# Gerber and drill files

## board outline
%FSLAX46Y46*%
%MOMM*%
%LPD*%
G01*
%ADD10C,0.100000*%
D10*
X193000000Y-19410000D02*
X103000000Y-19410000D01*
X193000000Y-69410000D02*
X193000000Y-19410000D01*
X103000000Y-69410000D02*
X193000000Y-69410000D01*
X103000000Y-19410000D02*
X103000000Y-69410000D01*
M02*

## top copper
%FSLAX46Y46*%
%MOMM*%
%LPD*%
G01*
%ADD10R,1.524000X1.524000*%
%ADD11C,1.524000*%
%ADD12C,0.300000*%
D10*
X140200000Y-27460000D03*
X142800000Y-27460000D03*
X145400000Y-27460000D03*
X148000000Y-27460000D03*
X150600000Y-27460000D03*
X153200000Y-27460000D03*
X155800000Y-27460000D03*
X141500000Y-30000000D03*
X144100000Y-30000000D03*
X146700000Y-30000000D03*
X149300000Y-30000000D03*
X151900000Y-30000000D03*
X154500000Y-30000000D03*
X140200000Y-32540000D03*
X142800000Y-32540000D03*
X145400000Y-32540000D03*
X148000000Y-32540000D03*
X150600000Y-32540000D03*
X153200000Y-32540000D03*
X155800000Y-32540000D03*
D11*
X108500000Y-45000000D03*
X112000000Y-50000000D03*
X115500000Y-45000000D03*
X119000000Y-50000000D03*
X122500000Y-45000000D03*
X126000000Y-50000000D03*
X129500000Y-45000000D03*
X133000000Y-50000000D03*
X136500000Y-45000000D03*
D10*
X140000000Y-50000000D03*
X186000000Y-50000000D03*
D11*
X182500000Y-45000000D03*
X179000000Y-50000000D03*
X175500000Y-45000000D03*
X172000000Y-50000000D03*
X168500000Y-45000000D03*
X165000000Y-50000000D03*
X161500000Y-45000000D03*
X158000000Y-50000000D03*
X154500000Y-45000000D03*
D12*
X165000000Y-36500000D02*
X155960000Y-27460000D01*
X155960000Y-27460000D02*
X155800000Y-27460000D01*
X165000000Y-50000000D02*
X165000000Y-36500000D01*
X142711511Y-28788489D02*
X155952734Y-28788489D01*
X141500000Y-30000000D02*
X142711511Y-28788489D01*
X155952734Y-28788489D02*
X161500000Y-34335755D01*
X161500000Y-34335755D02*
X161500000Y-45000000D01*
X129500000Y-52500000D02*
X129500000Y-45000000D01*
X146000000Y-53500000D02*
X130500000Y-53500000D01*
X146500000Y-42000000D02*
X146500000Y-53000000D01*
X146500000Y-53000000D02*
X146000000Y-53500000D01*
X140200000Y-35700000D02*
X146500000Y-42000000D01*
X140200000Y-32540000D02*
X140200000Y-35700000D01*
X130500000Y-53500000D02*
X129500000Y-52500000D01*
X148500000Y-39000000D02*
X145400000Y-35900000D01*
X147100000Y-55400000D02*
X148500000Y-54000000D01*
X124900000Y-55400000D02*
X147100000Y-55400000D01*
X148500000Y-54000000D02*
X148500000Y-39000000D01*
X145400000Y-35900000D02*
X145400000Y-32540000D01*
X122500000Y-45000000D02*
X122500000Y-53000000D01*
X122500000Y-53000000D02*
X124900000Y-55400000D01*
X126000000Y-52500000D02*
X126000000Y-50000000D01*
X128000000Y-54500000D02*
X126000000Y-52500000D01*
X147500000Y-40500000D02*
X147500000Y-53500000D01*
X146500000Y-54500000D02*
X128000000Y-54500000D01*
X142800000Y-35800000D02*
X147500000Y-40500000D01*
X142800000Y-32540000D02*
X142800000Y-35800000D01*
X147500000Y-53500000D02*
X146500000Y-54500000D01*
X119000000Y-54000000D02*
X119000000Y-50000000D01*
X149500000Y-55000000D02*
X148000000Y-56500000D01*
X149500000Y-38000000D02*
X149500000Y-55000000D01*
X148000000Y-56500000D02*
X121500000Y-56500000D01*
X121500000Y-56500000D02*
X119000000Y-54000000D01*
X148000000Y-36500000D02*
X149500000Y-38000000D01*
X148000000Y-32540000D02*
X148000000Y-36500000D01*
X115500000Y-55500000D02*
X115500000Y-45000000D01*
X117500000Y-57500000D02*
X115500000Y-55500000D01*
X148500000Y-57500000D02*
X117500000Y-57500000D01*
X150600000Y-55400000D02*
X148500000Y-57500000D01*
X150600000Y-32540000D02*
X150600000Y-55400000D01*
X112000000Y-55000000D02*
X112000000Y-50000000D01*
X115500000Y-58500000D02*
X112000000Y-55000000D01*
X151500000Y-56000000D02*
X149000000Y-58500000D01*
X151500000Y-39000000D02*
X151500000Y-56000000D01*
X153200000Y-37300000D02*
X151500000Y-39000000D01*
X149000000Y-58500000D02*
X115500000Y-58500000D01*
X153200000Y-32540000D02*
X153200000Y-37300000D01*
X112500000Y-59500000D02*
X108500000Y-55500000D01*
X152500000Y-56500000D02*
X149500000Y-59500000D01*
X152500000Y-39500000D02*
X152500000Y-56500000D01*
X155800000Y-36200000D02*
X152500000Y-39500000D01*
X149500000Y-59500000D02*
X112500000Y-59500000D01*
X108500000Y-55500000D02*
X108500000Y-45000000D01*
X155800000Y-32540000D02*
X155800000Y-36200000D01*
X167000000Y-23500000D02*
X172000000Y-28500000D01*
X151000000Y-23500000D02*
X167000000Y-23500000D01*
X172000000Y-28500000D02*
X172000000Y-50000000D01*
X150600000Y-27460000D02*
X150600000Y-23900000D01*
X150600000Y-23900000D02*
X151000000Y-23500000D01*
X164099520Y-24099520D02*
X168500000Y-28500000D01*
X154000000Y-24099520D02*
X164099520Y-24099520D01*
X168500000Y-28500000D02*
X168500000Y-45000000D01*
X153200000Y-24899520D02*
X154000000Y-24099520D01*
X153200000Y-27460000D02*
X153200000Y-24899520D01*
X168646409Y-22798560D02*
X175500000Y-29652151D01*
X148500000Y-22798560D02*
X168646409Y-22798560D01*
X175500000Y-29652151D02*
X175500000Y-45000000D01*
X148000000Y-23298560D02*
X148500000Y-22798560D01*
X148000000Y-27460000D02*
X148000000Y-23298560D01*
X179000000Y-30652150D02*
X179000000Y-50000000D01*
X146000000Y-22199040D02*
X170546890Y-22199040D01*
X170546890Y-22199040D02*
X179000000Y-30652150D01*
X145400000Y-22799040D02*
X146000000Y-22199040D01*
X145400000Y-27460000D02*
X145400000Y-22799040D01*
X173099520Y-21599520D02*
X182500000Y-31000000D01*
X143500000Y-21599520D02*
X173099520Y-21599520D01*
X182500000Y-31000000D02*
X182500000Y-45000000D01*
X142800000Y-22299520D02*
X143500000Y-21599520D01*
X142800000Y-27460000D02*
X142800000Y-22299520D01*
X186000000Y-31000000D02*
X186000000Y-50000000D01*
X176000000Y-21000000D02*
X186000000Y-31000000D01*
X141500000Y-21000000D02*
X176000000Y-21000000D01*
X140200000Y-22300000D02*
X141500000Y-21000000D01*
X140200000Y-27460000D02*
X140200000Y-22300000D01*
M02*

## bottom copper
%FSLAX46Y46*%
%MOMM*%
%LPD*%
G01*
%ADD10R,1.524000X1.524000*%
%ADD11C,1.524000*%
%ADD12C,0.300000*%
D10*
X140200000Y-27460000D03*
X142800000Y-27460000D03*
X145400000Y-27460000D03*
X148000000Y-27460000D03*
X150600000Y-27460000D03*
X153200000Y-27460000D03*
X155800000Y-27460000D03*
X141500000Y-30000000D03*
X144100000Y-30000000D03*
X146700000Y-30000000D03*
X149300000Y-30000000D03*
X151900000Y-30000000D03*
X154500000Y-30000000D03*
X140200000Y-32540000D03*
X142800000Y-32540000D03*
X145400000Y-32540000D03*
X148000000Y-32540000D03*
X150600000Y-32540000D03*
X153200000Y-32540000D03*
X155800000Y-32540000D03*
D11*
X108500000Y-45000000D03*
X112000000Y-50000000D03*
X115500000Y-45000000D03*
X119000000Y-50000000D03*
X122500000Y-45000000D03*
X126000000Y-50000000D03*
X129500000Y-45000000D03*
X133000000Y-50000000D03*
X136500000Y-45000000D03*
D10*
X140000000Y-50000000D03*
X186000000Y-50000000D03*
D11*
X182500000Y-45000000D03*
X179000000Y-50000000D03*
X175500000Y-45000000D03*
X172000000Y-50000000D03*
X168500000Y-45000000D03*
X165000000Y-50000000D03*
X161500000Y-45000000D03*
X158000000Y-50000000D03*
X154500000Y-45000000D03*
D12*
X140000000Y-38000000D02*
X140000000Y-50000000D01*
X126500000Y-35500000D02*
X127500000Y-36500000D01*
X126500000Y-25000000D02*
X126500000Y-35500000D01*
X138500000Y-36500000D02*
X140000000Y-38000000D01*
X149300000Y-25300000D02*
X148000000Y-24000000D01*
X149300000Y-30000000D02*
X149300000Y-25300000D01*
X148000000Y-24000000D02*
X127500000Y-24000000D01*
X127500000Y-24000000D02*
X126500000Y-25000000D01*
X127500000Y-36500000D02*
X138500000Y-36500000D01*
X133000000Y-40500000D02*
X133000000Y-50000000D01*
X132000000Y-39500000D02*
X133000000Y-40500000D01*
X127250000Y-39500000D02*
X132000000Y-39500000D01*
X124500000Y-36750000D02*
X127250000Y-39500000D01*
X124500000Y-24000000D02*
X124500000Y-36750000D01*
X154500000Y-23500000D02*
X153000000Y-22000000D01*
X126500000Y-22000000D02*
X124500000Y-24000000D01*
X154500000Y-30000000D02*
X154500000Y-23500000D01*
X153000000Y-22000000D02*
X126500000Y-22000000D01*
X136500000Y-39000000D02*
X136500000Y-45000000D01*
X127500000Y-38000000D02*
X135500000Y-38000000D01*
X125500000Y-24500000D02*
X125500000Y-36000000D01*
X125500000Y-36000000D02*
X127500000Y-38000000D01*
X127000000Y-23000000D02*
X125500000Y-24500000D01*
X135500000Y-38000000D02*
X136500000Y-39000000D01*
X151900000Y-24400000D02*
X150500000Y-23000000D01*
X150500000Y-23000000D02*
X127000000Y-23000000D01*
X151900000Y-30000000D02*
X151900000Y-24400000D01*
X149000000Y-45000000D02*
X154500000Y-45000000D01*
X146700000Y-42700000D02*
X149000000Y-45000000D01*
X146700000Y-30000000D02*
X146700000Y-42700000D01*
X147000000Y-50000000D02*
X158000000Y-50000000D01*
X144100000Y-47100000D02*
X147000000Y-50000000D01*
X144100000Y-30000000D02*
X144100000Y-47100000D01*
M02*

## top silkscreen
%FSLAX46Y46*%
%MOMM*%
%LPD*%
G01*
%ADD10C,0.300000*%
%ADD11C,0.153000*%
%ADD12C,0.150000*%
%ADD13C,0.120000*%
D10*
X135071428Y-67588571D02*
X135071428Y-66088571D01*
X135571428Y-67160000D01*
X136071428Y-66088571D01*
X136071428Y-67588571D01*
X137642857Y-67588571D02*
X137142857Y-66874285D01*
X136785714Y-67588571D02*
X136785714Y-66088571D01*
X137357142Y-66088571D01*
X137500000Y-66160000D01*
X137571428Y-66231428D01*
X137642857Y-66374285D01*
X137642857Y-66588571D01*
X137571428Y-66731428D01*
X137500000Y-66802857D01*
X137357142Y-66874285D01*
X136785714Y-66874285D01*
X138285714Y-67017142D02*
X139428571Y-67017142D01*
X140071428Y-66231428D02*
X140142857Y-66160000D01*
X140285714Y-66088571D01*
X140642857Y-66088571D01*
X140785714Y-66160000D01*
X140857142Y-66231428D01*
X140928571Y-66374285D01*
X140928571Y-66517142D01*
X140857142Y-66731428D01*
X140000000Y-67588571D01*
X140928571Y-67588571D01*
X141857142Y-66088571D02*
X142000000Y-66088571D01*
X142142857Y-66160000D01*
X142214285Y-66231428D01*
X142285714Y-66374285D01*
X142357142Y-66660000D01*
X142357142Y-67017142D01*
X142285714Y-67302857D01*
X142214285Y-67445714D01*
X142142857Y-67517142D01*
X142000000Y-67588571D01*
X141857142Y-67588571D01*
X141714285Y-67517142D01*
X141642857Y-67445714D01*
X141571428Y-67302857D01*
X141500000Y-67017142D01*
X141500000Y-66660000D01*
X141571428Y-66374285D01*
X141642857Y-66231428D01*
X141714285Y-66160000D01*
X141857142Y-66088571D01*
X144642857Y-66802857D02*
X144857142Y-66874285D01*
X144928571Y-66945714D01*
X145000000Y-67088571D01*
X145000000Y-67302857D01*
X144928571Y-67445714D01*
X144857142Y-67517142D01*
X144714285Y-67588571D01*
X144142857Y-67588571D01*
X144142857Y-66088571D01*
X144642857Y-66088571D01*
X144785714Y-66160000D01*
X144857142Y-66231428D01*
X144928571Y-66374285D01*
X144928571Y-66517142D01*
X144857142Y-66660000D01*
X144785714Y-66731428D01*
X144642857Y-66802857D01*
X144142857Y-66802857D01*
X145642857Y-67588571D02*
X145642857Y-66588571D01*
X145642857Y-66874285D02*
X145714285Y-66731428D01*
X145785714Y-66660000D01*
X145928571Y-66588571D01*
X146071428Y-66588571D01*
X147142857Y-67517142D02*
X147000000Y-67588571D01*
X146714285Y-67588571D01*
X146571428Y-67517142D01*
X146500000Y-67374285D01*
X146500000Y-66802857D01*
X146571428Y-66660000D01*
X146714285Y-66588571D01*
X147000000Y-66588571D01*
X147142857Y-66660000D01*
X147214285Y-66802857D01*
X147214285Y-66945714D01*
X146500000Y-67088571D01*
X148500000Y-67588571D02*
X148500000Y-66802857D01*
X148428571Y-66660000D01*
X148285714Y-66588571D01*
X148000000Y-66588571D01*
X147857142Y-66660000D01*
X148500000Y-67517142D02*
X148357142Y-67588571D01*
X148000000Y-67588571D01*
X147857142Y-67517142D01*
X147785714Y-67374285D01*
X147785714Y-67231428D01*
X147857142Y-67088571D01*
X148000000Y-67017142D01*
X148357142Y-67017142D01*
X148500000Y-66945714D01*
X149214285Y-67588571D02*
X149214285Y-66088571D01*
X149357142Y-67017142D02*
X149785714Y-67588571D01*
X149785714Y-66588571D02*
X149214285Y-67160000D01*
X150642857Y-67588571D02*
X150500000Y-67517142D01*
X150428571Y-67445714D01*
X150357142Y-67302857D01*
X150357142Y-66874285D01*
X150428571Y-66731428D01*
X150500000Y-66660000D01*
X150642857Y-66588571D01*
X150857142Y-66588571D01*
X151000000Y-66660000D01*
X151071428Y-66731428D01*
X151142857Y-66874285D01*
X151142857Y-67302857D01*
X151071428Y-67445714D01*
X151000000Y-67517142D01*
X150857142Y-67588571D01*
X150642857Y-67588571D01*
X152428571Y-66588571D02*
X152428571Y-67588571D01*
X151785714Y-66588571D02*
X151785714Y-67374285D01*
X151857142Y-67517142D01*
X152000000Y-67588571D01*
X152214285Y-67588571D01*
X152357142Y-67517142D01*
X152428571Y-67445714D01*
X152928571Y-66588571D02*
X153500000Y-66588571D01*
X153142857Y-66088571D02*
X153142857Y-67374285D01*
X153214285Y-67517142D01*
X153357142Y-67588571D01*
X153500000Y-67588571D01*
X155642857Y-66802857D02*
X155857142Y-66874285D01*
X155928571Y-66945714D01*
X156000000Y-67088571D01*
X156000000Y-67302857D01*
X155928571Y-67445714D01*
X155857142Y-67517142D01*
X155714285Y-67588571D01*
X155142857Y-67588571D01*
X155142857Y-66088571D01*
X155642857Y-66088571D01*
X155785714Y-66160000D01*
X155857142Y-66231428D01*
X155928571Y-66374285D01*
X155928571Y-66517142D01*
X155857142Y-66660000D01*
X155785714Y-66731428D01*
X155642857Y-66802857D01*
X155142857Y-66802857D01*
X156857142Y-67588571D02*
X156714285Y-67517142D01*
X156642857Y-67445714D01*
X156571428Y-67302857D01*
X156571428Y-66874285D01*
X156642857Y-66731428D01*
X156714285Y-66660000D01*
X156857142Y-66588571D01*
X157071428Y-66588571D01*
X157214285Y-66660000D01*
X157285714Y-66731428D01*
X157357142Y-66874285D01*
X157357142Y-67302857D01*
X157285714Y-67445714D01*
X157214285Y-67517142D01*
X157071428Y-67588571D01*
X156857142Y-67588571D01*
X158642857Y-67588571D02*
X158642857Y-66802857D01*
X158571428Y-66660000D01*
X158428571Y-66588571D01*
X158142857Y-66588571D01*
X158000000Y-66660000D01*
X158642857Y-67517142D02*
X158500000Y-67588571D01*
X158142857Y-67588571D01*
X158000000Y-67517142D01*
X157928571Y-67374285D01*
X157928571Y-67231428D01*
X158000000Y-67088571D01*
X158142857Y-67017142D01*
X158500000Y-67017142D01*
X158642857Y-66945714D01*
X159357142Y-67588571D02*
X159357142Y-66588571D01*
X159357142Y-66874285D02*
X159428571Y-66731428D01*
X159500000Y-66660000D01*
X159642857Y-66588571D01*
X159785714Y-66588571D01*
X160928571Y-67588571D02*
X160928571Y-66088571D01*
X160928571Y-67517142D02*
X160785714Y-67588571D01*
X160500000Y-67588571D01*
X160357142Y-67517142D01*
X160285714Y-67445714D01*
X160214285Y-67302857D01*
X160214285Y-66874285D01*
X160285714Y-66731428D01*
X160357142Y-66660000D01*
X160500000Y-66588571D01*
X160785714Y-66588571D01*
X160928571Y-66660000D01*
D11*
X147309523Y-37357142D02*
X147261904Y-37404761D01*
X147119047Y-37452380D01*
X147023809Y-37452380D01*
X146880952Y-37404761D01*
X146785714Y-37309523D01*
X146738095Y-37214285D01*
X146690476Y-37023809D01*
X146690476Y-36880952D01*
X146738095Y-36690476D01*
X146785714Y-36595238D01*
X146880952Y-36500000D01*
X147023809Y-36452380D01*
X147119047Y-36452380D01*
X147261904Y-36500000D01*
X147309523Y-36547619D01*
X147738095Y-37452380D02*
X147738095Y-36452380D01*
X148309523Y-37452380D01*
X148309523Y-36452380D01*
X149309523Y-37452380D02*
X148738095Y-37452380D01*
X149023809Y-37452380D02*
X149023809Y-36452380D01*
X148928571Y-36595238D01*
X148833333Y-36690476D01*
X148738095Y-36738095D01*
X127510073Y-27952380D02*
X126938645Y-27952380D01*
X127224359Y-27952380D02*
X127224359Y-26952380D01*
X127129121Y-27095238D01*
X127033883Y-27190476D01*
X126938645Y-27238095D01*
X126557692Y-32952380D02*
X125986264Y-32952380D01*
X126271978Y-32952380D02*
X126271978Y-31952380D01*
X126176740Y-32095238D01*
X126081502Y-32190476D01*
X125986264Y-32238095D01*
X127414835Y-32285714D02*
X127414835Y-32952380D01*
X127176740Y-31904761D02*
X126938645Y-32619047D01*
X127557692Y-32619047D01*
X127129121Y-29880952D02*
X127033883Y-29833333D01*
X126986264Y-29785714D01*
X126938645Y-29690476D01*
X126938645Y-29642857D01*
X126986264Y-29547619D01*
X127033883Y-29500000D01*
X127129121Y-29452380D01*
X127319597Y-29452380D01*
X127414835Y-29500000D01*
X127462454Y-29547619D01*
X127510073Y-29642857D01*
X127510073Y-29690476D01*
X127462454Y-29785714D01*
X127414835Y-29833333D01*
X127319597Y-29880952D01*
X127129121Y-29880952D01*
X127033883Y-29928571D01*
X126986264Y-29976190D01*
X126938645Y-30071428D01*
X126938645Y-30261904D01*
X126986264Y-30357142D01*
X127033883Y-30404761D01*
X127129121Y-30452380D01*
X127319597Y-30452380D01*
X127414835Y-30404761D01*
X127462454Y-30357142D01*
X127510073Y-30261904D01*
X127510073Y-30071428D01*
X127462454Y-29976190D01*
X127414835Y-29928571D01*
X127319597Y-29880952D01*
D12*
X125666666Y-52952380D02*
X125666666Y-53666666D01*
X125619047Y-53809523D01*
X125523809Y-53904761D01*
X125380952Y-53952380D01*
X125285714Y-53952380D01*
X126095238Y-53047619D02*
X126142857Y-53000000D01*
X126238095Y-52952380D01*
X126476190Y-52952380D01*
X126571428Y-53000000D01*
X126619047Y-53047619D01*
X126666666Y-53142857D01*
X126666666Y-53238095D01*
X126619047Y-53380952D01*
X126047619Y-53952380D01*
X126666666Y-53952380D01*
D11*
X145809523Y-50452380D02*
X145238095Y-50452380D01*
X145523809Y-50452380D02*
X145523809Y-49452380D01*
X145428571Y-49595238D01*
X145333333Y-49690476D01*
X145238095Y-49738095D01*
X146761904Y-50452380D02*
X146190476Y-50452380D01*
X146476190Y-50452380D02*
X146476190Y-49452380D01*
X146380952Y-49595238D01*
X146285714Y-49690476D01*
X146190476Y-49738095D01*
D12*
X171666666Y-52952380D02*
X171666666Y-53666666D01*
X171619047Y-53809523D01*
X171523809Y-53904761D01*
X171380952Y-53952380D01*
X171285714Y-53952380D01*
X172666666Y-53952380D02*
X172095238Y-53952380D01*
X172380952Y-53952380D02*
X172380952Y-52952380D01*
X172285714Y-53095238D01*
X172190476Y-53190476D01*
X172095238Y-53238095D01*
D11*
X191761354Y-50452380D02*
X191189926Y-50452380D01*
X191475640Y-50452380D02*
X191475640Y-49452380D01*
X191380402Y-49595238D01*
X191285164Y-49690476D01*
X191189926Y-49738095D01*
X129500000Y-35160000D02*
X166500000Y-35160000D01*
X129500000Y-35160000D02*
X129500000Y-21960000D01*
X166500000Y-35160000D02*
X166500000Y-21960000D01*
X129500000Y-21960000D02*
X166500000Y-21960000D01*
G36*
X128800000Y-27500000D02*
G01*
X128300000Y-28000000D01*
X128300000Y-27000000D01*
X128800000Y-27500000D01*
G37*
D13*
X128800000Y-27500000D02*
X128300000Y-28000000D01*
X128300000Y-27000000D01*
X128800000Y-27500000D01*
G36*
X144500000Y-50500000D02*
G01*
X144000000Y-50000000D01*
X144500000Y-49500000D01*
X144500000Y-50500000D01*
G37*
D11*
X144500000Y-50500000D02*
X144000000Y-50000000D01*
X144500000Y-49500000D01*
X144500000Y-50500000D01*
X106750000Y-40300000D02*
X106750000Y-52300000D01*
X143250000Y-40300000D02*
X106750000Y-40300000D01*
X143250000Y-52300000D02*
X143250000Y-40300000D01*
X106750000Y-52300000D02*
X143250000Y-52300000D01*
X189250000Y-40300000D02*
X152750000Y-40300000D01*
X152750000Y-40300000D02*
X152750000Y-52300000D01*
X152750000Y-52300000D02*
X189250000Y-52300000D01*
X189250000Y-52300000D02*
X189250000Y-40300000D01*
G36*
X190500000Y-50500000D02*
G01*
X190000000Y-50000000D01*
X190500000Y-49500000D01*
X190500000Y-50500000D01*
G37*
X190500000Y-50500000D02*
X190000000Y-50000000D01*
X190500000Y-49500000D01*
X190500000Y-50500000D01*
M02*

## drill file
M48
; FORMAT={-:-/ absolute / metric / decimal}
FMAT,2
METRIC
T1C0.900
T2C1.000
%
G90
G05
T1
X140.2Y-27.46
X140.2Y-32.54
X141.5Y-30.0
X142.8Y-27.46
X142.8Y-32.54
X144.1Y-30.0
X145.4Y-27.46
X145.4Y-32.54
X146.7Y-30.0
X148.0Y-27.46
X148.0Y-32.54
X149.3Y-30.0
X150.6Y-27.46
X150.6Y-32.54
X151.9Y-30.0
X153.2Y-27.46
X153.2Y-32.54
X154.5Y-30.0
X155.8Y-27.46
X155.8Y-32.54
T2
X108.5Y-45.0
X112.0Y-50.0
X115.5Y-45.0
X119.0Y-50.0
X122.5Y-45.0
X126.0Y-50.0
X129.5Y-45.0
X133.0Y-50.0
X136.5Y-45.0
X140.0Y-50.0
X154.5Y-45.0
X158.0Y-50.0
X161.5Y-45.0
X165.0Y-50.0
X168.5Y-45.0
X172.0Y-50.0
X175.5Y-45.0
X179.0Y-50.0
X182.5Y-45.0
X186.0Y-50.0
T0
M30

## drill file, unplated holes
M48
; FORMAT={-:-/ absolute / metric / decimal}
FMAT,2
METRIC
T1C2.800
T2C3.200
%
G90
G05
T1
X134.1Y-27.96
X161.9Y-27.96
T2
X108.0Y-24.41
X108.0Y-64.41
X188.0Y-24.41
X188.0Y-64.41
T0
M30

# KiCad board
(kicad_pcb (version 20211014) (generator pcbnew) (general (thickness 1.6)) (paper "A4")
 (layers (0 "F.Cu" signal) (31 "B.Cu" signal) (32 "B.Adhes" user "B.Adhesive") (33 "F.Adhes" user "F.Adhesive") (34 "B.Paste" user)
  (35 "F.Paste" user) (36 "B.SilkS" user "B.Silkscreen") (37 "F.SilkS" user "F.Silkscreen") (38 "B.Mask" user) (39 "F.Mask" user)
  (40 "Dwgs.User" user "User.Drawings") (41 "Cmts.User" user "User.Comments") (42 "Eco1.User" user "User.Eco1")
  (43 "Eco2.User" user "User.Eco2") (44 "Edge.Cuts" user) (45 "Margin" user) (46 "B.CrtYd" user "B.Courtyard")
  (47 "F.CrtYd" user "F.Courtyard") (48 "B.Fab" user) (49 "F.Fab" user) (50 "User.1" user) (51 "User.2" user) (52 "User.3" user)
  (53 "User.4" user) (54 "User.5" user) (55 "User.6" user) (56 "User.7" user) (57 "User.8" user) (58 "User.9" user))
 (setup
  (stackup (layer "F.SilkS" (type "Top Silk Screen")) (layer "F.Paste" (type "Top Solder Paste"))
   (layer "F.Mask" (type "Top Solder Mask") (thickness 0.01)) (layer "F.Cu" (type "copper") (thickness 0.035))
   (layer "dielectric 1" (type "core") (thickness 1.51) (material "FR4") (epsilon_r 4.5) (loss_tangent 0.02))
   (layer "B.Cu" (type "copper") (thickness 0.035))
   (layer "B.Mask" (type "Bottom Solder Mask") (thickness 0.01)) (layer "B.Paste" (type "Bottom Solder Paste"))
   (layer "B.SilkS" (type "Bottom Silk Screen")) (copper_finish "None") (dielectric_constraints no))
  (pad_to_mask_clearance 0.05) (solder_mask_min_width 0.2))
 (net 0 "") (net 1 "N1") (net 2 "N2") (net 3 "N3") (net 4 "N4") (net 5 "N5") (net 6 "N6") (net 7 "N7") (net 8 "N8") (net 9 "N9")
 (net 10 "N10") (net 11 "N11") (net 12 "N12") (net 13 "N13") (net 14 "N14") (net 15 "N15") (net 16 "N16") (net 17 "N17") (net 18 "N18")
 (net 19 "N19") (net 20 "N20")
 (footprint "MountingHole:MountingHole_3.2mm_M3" (layer "F.Cu") (at 188 64.41)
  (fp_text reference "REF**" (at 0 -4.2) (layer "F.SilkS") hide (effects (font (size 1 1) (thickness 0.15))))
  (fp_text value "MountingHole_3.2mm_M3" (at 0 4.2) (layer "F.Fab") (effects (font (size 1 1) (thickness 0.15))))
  (pad "" np_thru_hole circle (at 0 0) (size 3.2 3.2) (drill 3.2) (layers *.Cu *.Mask)))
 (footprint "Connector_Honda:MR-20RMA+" (layer "F.Cu") (at 148 30)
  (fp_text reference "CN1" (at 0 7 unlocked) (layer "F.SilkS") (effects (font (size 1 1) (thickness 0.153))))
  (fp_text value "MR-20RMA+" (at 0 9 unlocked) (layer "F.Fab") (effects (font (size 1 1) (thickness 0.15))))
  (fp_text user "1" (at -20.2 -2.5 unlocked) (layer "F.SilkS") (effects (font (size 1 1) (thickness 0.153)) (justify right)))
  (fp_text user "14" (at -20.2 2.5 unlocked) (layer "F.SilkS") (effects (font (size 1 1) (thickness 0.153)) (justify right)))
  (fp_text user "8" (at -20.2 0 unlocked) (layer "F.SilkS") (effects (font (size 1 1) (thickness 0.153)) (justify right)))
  (fp_line (start -18.5 5.16) (end 18.5 5.16) (layer "F.SilkS") (width 0.153))
  (fp_line (start -18.5 5.16) (end -18.5 -8.04) (layer "F.SilkS") (width 0.153))
  (fp_line (start 18.5 5.16) (end 18.5 -8.04) (layer "F.SilkS") (width 0.153))
  (fp_line (start -18.5 -8.04) (end 18.5 -8.04) (layer "F.SilkS") (width 0.153))
  (fp_poly (pts (xy -19.2 -2.5) (xy -19.7 -2) (xy -19.7 -3)) (layer "F.SilkS") (width 0.12) (fill solid))
  (pad "" np_thru_hole circle (at -13.9 -2.04) (size 2.8 2.8) (drill 2.8) (layers F&B.Cu *.Mask))
  (pad "" np_thru_hole circle (at 13.9 -2.04) (size 2.8 2.8) (drill 2.8) (layers F&B.Cu *.Mask))
  (pad "1" thru_hole rect (at -7.8 -2.54) (size 1.524 1.524) (drill 0.9) (layers *.Cu *.Mask) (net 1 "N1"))
  (pad "2" thru_hole rect (at -5.2 -2.54) (size 1.524 1.524) (drill 0.9) (layers *.Cu *.Mask) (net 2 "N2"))
  (pad "3" thru_hole rect (at -2.6 -2.54) (size 1.524 1.524) (drill 0.9) (layers *.Cu *.Mask) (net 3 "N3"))
  (pad "4" thru_hole rect (at 0 -2.54) (size 1.524 1.524) (drill 0.9) (layers *.Cu *.Mask) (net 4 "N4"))
  (pad "5" thru_hole rect (at 2.6 -2.54) (size 1.524 1.524) (drill 0.9) (layers *.Cu *.Mask) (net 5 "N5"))
  (pad "6" thru_hole rect (at 5.2 -2.54) (size 1.524 1.524) (drill 0.9) (layers *.Cu *.Mask) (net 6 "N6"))
  (pad "7" thru_hole rect (at 7.8 -2.54) (size 1.524 1.524) (drill 0.9) (layers *.Cu *.Mask) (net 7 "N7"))
  (pad "8" thru_hole rect (at -6.5 0) (size 1.524 1.524) (drill 0.9) (layers *.Cu *.Mask) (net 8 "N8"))
  (pad "9" thru_hole rect (at -3.9 0) (size 1.524 1.524) (drill 0.9) (layers *.Cu *.Mask) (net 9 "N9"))
  (pad "10" thru_hole rect (at -1.3 0) (size 1.524 1.524) (drill 0.9) (layers *.Cu *.Mask) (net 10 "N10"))
  (pad "11" thru_hole rect (at 1.3 0) (size 1.524 1.524) (drill 0.9) (layers *.Cu *.Mask) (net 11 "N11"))
  (pad "12" thru_hole rect (at 3.9 0) (size 1.524 1.524) (drill 0.9) (layers *.Cu *.Mask) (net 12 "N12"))
  (pad "13" thru_hole rect (at 6.5 0) (size 1.524 1.524) (drill 0.9) (layers *.Cu *.Mask) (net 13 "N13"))
  (pad "14" thru_hole rect (at -7.8 2.54) (size 1.524 1.524) (drill 0.9) (layers *.Cu *.Mask) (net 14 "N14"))
  (pad "15" thru_hole rect (at -5.2 2.54) (size 1.524 1.524) (drill 0.9) (layers *.Cu *.Mask) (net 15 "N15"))
  (pad "16" thru_hole rect (at -2.6 2.54) (size 1.524 1.524) (drill 0.9) (layers *.Cu *.Mask) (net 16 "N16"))
  (pad "17" thru_hole rect (at 0 2.54) (size 1.524 1.524) (drill 0.9) (layers *.Cu *.Mask) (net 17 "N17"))
  (pad "18" thru_hole rect (at 2.6 2.54) (size 1.524 1.524) (drill 0.9) (layers *.Cu *.Mask) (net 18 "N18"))
  (pad "19" thru_hole rect (at 5.2 2.54) (size 1.524 1.524) (drill 0.9) (layers *.Cu *.Mask) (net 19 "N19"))
  (pad "20" thru_hole rect (at 7.8 2.54) (size 1.524 1.524) (drill 0.9) (layers *.Cu *.Mask) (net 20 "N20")))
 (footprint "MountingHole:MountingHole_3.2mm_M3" (layer "F.Cu") (at 108 64.41)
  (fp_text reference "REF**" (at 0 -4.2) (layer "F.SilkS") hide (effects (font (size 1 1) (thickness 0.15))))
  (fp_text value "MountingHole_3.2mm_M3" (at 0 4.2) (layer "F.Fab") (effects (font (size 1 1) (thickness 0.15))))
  (pad "" np_thru_hole circle (at 0 0) (size 3.2 3.2) (drill 3.2) (layers *.Cu *.Mask)))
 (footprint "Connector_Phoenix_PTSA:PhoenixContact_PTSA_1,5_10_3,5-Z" (layer "F.Cu") (at 140 50 180)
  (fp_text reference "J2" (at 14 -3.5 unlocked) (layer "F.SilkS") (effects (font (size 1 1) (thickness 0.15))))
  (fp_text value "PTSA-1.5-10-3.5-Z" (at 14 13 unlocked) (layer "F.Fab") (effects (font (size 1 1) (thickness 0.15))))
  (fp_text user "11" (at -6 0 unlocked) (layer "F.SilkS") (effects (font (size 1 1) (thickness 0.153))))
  (fp_line (start 33.25 -2.3) (end -3.25 -2.3) (layer "F.SilkS") (width 0.153))
  (fp_line (start -3.25 -2.3) (end -3.25 9.7) (layer "F.SilkS") (width 0.153))
  (fp_line (start -3.25 9.7) (end 33.25 9.7) (layer "F.SilkS") (width 0.153))
  (fp_line (start 33.25 9.7) (end 33.25 -2.3) (layer "F.SilkS") (width 0.153))
  (fp_poly (pts (xy -4 0) (xy -4.5 0.5) (xy -4.5 -0.5)) (layer "F.SilkS") (width 0.153) (fill solid))
  (pad "1" thru_hole rect (at 0 0 180) (size 1.524 1.524) (drill 1) (layers *.Cu *.Mask) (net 11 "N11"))
  (pad "2" thru_hole circle (at 3.5 5 180) (size 1.524 1.524) (drill 1) (layers *.Cu *.Mask) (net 12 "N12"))
  (pad "3" thru_hole circle (at 7 0 180) (size 1.524 1.524) (drill 1) (layers *.Cu *.Mask) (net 13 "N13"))
  (pad "4" thru_hole circle (at 10.5 5 180) (size 1.524 1.524) (drill 1) (layers *.Cu *.Mask) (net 14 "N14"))
  (pad "5" thru_hole circle (at 14 0 180) (size 1.524 1.524) (drill 1) (layers *.Cu *.Mask) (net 15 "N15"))
  (pad "6" thru_hole circle (at 17.5 5 180) (size 1.524 1.524) (drill 1) (layers *.Cu *.Mask) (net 16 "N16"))
  (pad "7" thru_hole circle (at 21 0 180) (size 1.524 1.524) (drill 1) (layers *.Cu *.Mask) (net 17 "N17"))
  (pad "8" thru_hole circle (at 24.5 5 180) (size 1.524 1.524) (drill 1) (layers *.Cu *.Mask) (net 18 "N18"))
  (pad "9" thru_hole circle (at 28 0 180) (size 1.524 1.524) (drill 1) (layers *.Cu *.Mask) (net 19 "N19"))
  (pad "10" thru_hole circle (at 31.5 5 180) (size 1.524 1.524) (drill 1) (layers *.Cu *.Mask) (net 20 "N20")))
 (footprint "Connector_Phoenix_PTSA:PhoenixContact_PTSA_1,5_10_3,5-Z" (layer "F.Cu") (at 186 50 180)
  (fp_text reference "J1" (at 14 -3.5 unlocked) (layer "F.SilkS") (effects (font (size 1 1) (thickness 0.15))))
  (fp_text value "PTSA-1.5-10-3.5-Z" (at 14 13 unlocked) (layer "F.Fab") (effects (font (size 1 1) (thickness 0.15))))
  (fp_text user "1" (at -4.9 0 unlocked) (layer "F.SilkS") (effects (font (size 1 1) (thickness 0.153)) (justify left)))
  (fp_line (start -3.25 9.7) (end 33.25 9.7) (layer "F.SilkS") (width 0.153))
  (fp_line (start 33.25 9.7) (end 33.25 -2.3) (layer "F.SilkS") (width 0.153))
  (fp_line (start 33.25 -2.3) (end -3.25 -2.3) (layer "F.SilkS") (width 0.153))
  (fp_line (start -3.25 -2.3) (end -3.25 9.7) (layer "F.SilkS") (width 0.153))
  (fp_poly (pts (xy -4 0) (xy -4.5 0.5) (xy -4.5 -0.5)) (layer "F.SilkS") (width 0.153) (fill solid))
  (pad "1" thru_hole rect (at 0 0 180) (size 1.524 1.524) (drill 1) (layers *.Cu *.Mask) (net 1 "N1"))
  (pad "2" thru_hole circle (at 3.5 5 180) (size 1.524 1.524) (drill 1) (layers *.Cu *.Mask) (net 2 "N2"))
  (pad "3" thru_hole circle (at 7 0 180) (size 1.524 1.524) (drill 1) (layers *.Cu *.Mask) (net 3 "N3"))
  (pad "4" thru_hole circle (at 10.5 5 180) (size 1.524 1.524) (drill 1) (layers *.Cu *.Mask) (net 4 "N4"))
  (pad "5" thru_hole circle (at 14 0 180) (size 1.524 1.524) (drill 1) (layers *.Cu *.Mask) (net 5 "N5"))
  (pad "6" thru_hole circle (at 17.5 5 180) (size 1.524 1.524) (drill 1) (layers *.Cu *.Mask) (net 6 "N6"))
  (pad "7" thru_hole circle (at 21 0 180) (size 1.524 1.524) (drill 1) (layers *.Cu *.Mask) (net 7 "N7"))
  (pad "8" thru_hole circle (at 24.5 5 180) (size 1.524 1.524) (drill 1) (layers *.Cu *.Mask) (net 8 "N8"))
  (pad "9" thru_hole circle (at 28 0 180) (size 1.524 1.524) (drill 1) (layers *.Cu *.Mask) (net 9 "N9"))
  (pad "10" thru_hole circle (at 31.5 5 180) (size 1.524 1.524) (drill 1) (layers *.Cu *.Mask) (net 10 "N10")))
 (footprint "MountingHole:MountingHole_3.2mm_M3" (layer "F.Cu") (at 188 24.41)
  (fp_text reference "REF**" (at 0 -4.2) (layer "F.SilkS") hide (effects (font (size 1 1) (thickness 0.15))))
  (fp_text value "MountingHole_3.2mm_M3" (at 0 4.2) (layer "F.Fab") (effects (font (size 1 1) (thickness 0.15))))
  (pad "" np_thru_hole circle (at 0 0) (size 3.2 3.2) (drill 3.2) (layers *.Cu *.Mask)))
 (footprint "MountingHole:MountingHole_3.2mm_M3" (layer "F.Cu") (at 108 24.41)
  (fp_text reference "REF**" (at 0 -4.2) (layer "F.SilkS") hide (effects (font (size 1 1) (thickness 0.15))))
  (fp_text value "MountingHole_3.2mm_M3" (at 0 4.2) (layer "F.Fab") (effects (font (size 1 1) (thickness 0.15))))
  (pad "" np_thru_hole circle (at 0 0) (size 3.2 3.2) (drill 3.2) (layers *.Cu *.Mask)))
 (gr_line (start 193 19.41) (end 103 19.41) (layer "Edge.Cuts") (width 0.1))
 (gr_line (start 193 69.41) (end 193 19.41) (layer "Edge.Cuts") (width 0.1))
 (gr_line (start 103 69.41) (end 193 69.41) (layer "Edge.Cuts") (width 0.1))
 (gr_line (start 103 19.41) (end 103 69.41) (layer "Edge.Cuts") (width 0.1))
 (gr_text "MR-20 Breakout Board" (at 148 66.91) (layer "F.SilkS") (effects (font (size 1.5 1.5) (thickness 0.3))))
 (segment (start 186 31) (end 186 50) (width 0.3) (layer "F.Cu") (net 1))
 (segment (start 176 21) (end 186 31) (width 0.3) (layer "F.Cu") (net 1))
 (segment (start 140.2 22.3) (end 141.5 21) (width 0.3) (layer "F.Cu") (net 1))
 (segment (start 140.2 27.46) (end 140.2 22.3) (width 0.3) (layer "F.Cu") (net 1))
 (segment (start 141.5 21) (end 176 21) (width 0.3) (layer "F.Cu") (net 1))
 (segment (start 173.09952 21.59952) (end 182.5 31) (width 0.3) (layer "F.Cu") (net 2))
 (segment (start 142.8 22.29952) (end 143.5 21.59952) (width 0.3) (layer "F.Cu") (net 2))
 (segment (start 143.5 21.59952) (end 173.09952 21.59952) (width 0.3) (layer "F.Cu") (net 2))
 (segment (start 182.5 31) (end 182.5 45) (width 0.3) (layer "F.Cu") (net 2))
 (segment (start 142.8 27.46) (end 142.8 22.29952) (width 0.3) (layer "F.Cu") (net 2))
 (segment (start 145.4 27.46) (end 145.4 22.79904) (width 0.3) (layer "F.Cu") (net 3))
 (segment (start 146 22.19904) (end 170.54689 22.19904) (width 0.3) (layer "F.Cu") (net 3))
 (segment (start 145.4 22.79904) (end 146 22.19904) (width 0.3) (layer "F.Cu") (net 3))
 (segment (start 170.54689 22.19904) (end 179 30.65215) (width 0.3) (layer "F.Cu") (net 3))
 (segment (start 179 30.65215) (end 179 50) (width 0.3) (layer "F.Cu") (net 3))
 (segment (start 148.5 22.79856) (end 168.646409 22.79856) (width 0.3) (layer "F.Cu") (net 4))
 (segment (start 148 23.29856) (end 148.5 22.79856) (width 0.3) (layer "F.Cu") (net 4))
 (segment (start 148 27.46) (end 148 23.29856) (width 0.3) (layer "F.Cu") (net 4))
 (segment (start 175.5 29.652151) (end 175.5 45) (width 0.3) (layer "F.Cu") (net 4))
 (segment (start 168.646409 22.79856) (end 175.5 29.652151) (width 0.3) (layer "F.Cu") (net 4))
 (segment (start 150.6 23.9) (end 151 23.5) (width 0.3) (layer "F.Cu") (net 5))
 (segment (start 172 28.5) (end 172 50) (width 0.3) (layer "F.Cu") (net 5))
 (segment (start 167 23.5) (end 172 28.5) (width 0.3) (layer "F.Cu") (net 5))
 (segment (start 150.6 27.46) (end 150.6 23.9) (width 0.3) (layer "F.Cu") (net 5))
 (segment (start 151 23.5) (end 167 23.5) (width 0.3) (layer "F.Cu") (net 5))
 (segment (start 153.2 27.46) (end 153.2 24.89952) (width 0.3) (layer "F.Cu") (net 6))
 (segment (start 168.5 28.5) (end 168.5 45) (width 0.3) (layer "F.Cu") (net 6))
 (segment (start 164.09952 24.09952) (end 168.5 28.5) (width 0.3) (layer "F.Cu") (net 6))
 (segment (start 154 24.09952) (end 164.09952 24.09952) (width 0.3) (layer "F.Cu") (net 6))
 (segment (start 153.2 24.89952) (end 154 24.09952) (width 0.3) (layer "F.Cu") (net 6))
 (segment (start 155.96 27.46) (end 155.8 27.46) (width 0.3) (layer "F.Cu") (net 7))
 (segment (start 165 50) (end 165 36.5) (width 0.3) (layer "F.Cu") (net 7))
 (segment (start 165 36.5) (end 155.96 27.46) (width 0.3) (layer "F.Cu") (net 7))
 (segment (start 161.5 34.335755) (end 161.5 45) (width 0.3) (layer "F.Cu") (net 8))
 (segment (start 141.5 30) (end 142.711511 28.788489) (width 0.3) (layer "F.Cu") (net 8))
 (segment (start 142.711511 28.788489) (end 155.952734 28.788489) (width 0.3) (layer "F.Cu") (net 8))
 (segment (start 155.952734 28.788489) (end 161.5 34.335755) (width 0.3) (layer "F.Cu") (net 8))
 (segment (start 144.1 47.1) (end 147 50) (width 0.3) (layer "B.Cu") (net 9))
 (segment (start 144.1 30) (end 144.1 47.1) (width 0.3) (layer "B.Cu") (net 9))
 (segment (start 147 50) (end 158 50) (width 0.3) (layer "B.Cu") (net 9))
 (segment (start 146.7 30) (end 146.7 42.7) (width 0.3) (layer "B.Cu") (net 10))
 (segment (start 149 45) (end 154.5 45) (width 0.3) (layer "B.Cu") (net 10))
 (segment (start 146.7 42.7) (end 149 45) (width 0.3) (layer "B.Cu") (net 10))
 (segment (start 127.5 24) (end 126.5 25) (width 0.3) (layer "B.Cu") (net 11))
 (segment (start 149.3 30) (end 149.3 25.3) (width 0.3) (layer "B.Cu") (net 11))
 (segment (start 126.5 25) (end 126.5 35.5) (width 0.3) (layer "B.Cu") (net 11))
 (segment (start 126.5 35.5) (end 127.5 36.5) (width 0.3) (layer "B.Cu") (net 11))
 (segment (start 140 38) (end 140 50) (width 0.3) (layer "B.Cu") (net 11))
 (segment (start 148 24) (end 127.5 24) (width 0.3) (layer "B.Cu") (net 11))
 (segment (start 138.5 36.5) (end 140 38) (width 0.3) (layer "B.Cu") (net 11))
 (segment (start 127.5 36.5) (end 138.5 36.5) (width 0.3) (layer "B.Cu") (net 11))
 (segment (start 149.3 25.3) (end 148 24) (width 0.3) (layer "B.Cu") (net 11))
 (segment (start 127 23) (end 125.5 24.5) (width 0.3) (layer "B.Cu") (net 12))
 (segment (start 125.5 36) (end 127.5 38) (width 0.3) (layer "B.Cu") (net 12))
 (segment (start 150.5 23) (end 127 23) (width 0.3) (layer "B.Cu") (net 12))
 (segment (start 125.5 24.5) (end 125.5 36) (width 0.3) (layer "B.Cu") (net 12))
 (segment (start 135.5 38) (end 136.5 39) (width 0.3) (layer "B.Cu") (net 12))
 (segment (start 151.9 24.4) (end 150.5 23) (width 0.3) (layer "B.Cu") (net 12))
 (segment (start 127.5 38) (end 135.5 38) (width 0.3) (layer "B.Cu") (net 12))
 (segment (start 151.9 30) (end 151.9 24.4) (width 0.3) (layer "B.Cu") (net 12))
 (segment (start 136.5 39) (end 136.5 45) (width 0.3) (layer "B.Cu") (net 12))
 (segment (start 133 40.5) (end 133 50) (width 0.3) (layer "B.Cu") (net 13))
 (segment (start 127.25 39.5) (end 132 39.5) (width 0.3) (layer "B.Cu") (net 13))
 (segment (start 126.5 22) (end 124.5 24) (width 0.3) (layer "B.Cu") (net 13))
 (segment (start 154.5 30) (end 154.5 23.5) (width 0.3) (layer "B.Cu") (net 13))
 (segment (start 154.5 23.5) (end 153 22) (width 0.3) (layer "B.Cu") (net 13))
 (segment (start 124.5 24) (end 124.5 36.75) (width 0.3) (layer "B.Cu") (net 13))
 (segment (start 132 39.5) (end 133 40.5) (width 0.3) (layer "B.Cu") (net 13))
 (segment (start 124.5 36.75) (end 127.25 39.5) (width 0.3) (layer "B.Cu") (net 13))
 (segment (start 153 22) (end 126.5 22) (width 0.3) (layer "B.Cu") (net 13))
 (segment (start 140.2 32.54) (end 140.2 35.7) (width 0.3) (layer "F.Cu") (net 14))
 (segment (start 129.5 52.5) (end 129.5 45) (width 0.3) (layer "F.Cu") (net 14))
 (segment (start 146.5 53) (end 146 53.5) (width 0.3) (layer "F.Cu") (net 14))
 (segment (start 140.2 35.7) (end 146.5 42) (width 0.3) (layer "F.Cu") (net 14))
 (segment (start 130.5 53.5) (end 129.5 52.5) (width 0.3) (layer "F.Cu") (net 14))
 (segment (start 146 53.5) (end 130.5 53.5) (width 0.3) (layer "F.Cu") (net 14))
 (segment (start 146.5 42) (end 146.5 53) (width 0.3) (layer "F.Cu") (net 14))
 (segment (start 126 52.5) (end 126 50) (width 0.3) (layer "F.Cu") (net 15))
 (segment (start 147.5 40.5) (end 147.5 53.5) (width 0.3) (layer "F.Cu") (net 15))
 (segment (start 128 54.5) (end 126 52.5) (width 0.3) (layer "F.Cu") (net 15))
 (segment (start 147.5 53.5) (end 146.5 54.5) (width 0.3) (layer "F.Cu") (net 15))
 (segment (start 142.8 35.8) (end 147.5 40.5) (width 0.3) (layer "F.Cu") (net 15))
 (segment (start 146.5 54.5) (end 128 54.5) (width 0.3) (layer "F.Cu") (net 15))
 (segment (start 142.8 32.54) (end 142.8 35.8) (width 0.3) (layer "F.Cu") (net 15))
 (segment (start 124.9 55.4) (end 147.1 55.4) (width 0.3) (layer "F.Cu") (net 16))
 (segment (start 122.5 45) (end 122.5 53) (width 0.3) (layer "F.Cu") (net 16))
 (segment (start 145.4 35.9) (end 145.4 32.54) (width 0.3) (layer "F.Cu") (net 16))
 (segment (start 122.5 53) (end 124.9 55.4) (width 0.3) (layer "F.Cu") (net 16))
 (segment (start 148.5 39) (end 145.4 35.9) (width 0.3) (layer "F.Cu") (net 16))
 (segment (start 147.1 55.4) (end 148.5 54) (width 0.3) (layer "F.Cu") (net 16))
 (segment (start 148.5 54) (end 148.5 39) (width 0.3) (layer "F.Cu") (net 16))
 (segment (start 149.5 38) (end 149.5 55) (width 0.3) (layer "F.Cu") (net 17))
 (segment (start 121.5 56.5) (end 119 54) (width 0.3) (layer "F.Cu") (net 17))
 (segment (start 149.5 55) (end 148 56.5) (width 0.3) (layer "F.Cu") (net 17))
 (segment (start 148 36.5) (end 149.5 38) (width 0.3) (layer "F.Cu") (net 17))
 (segment (start 148 32.54) (end 148 36.5) (width 0.3) (layer "F.Cu") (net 17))
 (segment (start 119 54) (end 119 50) (width 0.3) (layer "F.Cu") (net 17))
 (segment (start 148 56.5) (end 121.5 56.5) (width 0.3) (layer "F.Cu") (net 17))
 (segment (start 115.5 55.5) (end 115.5 45) (width 0.3) (layer "F.Cu") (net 18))
 (segment (start 150.6 55.4) (end 148.5 57.5) (width 0.3) (layer "F.Cu") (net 18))
 (segment (start 148.5 57.5) (end 117.5 57.5) (width 0.3) (layer "F.Cu") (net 18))
 (segment (start 117.5 57.5) (end 115.5 55.5) (width 0.3) (layer "F.Cu") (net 18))
 (segment (start 150.6 32.54) (end 150.6 55.4) (width 0.3) (layer "F.Cu") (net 18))
 (segment (start 115.5 58.5) (end 112 55) (width 0.3) (layer "F.Cu") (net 19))
 (segment (start 151.5 56) (end 149 58.5) (width 0.3) (layer "F.Cu") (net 19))
 (segment (start 153.2 37.3) (end 151.5 39) (width 0.3) (layer "F.Cu") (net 19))
 (segment (start 149 58.5) (end 115.5 58.5) (width 0.3) (layer "F.Cu") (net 19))
 (segment (start 151.5 39) (end 151.5 56) (width 0.3) (layer "F.Cu") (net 19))
 (segment (start 112 55) (end 112 50) (width 0.3) (layer "F.Cu") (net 19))
 (segment (start 153.2 32.54) (end 153.2 37.3) (width 0.3) (layer "F.Cu") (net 19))
 (segment (start 155.8 32.54) (end 155.8 36.2) (width 0.3) (layer "F.Cu") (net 20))
 (segment (start 152.5 56.5) (end 149.5 59.5) (width 0.3) (layer "F.Cu") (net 20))
 (segment (start 152.5 39.5) (end 152.5 56.5) (width 0.3) (layer "F.Cu") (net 20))
 (segment (start 149.5 59.5) (end 112.5 59.5) (width 0.3) (layer "F.Cu") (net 20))
 (segment (start 112.5 59.5) (end 108.5 55.5) (width 0.3) (layer "F.Cu") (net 20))
 (segment (start 108.5 55.5) (end 108.5 45) (width 0.3) (layer "F.Cu") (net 20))
 (segment (start 155.8 36.2) (end 152.5 39.5) (width 0.3) (layer "F.Cu") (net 20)))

